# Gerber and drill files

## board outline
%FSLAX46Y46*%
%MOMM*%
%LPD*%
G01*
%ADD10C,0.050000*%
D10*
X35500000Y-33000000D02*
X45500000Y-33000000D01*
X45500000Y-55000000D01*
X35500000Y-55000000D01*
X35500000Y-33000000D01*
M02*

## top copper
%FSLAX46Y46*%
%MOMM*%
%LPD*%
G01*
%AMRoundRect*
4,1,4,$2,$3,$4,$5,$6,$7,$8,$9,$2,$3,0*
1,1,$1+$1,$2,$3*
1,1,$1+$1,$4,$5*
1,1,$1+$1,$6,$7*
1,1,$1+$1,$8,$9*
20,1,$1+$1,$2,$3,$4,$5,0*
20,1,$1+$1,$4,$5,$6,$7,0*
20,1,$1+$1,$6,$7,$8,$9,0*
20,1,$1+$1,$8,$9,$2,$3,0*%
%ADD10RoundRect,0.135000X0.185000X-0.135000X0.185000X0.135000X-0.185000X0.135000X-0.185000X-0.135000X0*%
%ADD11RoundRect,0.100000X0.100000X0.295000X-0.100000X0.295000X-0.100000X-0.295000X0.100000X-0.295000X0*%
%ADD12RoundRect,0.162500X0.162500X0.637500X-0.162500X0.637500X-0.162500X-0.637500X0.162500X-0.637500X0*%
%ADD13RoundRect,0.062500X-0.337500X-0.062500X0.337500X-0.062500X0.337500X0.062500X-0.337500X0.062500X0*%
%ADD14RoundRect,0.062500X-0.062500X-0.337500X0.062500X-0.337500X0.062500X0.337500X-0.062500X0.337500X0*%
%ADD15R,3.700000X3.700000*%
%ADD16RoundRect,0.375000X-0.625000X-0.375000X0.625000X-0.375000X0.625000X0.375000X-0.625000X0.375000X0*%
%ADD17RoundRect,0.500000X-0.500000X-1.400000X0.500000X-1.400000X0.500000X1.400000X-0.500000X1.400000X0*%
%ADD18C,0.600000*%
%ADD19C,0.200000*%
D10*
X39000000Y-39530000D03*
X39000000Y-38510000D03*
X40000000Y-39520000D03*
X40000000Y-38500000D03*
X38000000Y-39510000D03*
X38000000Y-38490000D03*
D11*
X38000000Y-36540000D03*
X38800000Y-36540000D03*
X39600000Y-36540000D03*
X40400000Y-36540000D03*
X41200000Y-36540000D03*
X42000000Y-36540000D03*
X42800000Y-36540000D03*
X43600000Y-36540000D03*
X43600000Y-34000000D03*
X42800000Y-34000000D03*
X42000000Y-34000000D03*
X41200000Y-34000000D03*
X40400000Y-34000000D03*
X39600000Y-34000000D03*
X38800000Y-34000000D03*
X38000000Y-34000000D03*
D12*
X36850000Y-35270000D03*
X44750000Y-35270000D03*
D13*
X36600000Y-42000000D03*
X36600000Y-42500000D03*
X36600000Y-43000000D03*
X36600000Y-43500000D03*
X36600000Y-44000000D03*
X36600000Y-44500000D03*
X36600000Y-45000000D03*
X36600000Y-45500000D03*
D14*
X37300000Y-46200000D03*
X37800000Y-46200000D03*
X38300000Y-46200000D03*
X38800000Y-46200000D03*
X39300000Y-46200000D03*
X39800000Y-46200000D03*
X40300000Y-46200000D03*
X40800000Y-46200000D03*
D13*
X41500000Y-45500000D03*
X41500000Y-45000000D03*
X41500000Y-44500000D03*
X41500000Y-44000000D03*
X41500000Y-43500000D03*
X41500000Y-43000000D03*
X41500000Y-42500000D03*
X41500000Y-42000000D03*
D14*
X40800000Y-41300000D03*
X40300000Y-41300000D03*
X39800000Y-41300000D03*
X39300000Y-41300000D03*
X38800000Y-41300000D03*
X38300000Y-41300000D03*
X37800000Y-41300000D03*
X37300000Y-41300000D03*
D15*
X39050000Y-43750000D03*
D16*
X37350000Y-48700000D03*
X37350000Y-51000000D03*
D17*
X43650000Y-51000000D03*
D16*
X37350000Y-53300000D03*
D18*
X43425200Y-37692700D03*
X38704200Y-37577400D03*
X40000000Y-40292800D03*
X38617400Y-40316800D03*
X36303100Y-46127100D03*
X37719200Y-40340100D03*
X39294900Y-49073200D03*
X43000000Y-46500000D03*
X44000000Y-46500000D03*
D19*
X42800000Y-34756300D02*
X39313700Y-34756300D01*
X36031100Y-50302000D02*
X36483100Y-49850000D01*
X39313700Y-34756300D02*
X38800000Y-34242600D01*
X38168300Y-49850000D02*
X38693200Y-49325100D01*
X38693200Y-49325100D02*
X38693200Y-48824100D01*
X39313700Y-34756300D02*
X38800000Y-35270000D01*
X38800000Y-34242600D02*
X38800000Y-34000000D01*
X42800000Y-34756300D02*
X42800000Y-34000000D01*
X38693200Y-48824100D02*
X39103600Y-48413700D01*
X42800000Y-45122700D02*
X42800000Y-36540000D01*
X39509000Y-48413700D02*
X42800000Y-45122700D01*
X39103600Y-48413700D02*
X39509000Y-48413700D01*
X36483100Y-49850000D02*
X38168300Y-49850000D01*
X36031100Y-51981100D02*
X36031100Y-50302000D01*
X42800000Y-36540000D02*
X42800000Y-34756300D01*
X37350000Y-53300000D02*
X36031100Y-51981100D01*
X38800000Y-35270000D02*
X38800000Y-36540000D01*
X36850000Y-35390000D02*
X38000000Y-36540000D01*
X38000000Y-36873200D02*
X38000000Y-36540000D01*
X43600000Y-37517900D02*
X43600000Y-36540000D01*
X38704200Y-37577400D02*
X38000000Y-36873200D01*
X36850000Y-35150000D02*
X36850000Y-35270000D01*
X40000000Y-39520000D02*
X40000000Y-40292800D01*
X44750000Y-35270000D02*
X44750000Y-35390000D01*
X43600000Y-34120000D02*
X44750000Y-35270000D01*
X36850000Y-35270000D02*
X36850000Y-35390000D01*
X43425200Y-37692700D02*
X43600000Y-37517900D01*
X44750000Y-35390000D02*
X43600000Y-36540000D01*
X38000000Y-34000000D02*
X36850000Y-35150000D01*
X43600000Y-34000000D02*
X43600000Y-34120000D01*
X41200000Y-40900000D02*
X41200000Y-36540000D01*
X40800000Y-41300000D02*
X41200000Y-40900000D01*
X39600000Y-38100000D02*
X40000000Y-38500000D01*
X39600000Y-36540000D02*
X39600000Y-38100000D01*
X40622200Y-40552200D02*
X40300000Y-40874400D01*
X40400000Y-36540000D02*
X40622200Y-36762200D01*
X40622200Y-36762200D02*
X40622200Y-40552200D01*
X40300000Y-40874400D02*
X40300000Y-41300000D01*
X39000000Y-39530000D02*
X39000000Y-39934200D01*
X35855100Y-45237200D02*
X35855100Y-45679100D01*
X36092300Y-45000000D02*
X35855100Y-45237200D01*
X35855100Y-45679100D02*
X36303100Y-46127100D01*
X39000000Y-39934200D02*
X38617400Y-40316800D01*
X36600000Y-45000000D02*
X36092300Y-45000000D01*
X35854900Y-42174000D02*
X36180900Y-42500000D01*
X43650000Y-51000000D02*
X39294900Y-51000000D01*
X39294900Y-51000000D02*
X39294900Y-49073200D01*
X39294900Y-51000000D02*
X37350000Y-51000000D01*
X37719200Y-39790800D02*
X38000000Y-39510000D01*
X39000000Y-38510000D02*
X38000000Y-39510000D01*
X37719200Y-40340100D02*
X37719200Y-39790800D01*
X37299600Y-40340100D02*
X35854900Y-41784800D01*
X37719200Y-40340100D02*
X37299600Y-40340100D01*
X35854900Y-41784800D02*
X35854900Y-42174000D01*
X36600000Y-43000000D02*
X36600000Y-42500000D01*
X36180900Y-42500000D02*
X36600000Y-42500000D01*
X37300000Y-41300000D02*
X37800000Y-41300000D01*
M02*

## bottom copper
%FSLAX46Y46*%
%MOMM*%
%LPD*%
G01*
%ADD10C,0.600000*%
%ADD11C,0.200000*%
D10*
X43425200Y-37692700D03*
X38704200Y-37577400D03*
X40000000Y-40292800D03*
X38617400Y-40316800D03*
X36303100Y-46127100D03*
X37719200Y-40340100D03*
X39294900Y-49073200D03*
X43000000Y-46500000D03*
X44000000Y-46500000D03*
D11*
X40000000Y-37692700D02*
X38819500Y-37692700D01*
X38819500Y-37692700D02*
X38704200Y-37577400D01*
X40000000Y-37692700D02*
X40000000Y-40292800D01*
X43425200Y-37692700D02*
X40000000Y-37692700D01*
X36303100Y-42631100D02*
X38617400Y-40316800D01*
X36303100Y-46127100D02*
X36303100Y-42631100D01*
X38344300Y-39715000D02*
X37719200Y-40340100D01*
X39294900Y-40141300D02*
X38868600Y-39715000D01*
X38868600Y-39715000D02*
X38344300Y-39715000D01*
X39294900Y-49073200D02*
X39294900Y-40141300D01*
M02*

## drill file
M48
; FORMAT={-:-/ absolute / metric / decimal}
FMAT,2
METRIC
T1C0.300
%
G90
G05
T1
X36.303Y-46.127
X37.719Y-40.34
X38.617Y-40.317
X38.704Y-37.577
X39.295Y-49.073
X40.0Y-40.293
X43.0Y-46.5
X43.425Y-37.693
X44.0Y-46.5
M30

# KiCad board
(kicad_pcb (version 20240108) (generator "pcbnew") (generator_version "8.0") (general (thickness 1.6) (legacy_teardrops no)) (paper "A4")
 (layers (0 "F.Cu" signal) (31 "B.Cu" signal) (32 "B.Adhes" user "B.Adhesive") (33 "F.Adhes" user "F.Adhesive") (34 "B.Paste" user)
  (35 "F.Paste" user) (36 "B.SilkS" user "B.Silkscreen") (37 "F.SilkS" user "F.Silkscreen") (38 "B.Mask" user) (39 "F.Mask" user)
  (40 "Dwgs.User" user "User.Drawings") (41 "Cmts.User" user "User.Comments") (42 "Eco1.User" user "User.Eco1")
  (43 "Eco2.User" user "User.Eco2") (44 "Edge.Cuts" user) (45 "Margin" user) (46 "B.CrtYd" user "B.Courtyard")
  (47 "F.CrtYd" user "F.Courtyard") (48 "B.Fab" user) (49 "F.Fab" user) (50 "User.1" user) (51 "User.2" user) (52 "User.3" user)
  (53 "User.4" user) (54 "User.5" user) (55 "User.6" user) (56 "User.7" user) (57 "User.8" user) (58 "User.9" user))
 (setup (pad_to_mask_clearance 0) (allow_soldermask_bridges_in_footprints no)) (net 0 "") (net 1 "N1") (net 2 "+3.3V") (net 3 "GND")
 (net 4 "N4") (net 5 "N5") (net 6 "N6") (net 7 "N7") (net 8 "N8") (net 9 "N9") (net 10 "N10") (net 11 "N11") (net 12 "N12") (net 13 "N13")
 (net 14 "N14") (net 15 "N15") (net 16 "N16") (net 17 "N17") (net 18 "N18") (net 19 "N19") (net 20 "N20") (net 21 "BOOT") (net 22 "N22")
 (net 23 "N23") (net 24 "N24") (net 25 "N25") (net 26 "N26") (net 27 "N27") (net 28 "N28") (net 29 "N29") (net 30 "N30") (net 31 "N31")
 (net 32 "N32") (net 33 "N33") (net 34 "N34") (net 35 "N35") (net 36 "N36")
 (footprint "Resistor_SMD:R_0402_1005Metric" (layer "F.Cu") (at 39 39.02 90)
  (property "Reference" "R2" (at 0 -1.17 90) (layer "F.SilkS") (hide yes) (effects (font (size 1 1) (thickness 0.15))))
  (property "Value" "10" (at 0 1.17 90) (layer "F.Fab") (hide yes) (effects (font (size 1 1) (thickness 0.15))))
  (pad "1" smd roundrect (at -0.51 0 90) (size 0.54 0.64) (layers "F.Cu" "F.Paste" "F.Mask") (roundrect_rratio 0.25) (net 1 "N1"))
  (pad "2" smd roundrect (at 0.51 0 90) (size 0.54 0.64) (layers "F.Cu" "F.Paste" "F.Mask") (roundrect_rratio 0.25) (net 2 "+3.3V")))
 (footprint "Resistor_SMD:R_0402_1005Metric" (layer "F.Cu") (at 40 39.01 90)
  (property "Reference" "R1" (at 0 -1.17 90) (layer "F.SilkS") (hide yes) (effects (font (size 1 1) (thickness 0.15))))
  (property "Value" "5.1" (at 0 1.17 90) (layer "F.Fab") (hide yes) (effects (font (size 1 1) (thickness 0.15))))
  (pad "1" smd roundrect (at -0.51 0 90) (size 0.54 0.64) (layers "F.Cu" "F.Paste" "F.Mask") (roundrect_rratio 0.25) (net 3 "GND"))
  (pad "2" smd roundrect (at 0.51 0 90) (size 0.54 0.64) (layers "F.Cu" "F.Paste" "F.Mask") (roundrect_rratio 0.25) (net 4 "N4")))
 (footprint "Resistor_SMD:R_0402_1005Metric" (layer "F.Cu") (at 38 39 90)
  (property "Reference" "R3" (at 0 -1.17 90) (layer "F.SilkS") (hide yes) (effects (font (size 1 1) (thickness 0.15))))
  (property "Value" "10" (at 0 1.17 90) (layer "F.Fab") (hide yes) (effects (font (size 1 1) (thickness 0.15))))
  (pad "1" smd roundrect (at -0.51 0 90) (size 0.54 0.64) (layers "F.Cu" "F.Paste" "F.Mask") (roundrect_rratio 0.25) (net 2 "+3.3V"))
  (pad "2" smd roundrect (at 0.51 0 90) (size 0.54 0.64) (layers "F.Cu" "F.Paste" "F.Mask") (roundrect_rratio 0.25) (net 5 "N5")))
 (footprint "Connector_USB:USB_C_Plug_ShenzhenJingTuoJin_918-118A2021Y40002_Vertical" (layer "F.Cu") (at 40.8 35.27 90)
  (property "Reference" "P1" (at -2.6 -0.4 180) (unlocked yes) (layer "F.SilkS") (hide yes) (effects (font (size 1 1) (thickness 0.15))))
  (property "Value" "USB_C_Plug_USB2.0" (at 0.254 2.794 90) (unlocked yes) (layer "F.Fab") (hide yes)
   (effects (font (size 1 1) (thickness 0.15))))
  (pad "A1" smd roundrect (at -1.27 -2.8 180) (size 0.4 0.79) (layers "F.Cu" "F.Paste" "F.Mask") (roundrect_rratio 0.25) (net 3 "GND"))
  (pad "A4" smd roundrect (at -1.27 -2 180) (size 0.4 0.79) (layers "F.Cu" "F.Paste" "F.Mask") (roundrect_rratio 0.25) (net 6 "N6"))
  (pad "A5" smd roundrect (at -1.27 -1.2 180) (size 0.4 0.79) (layers "F.Cu" "F.Paste" "F.Mask") (roundrect_rratio 0.25) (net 4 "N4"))
  (pad "A6" smd roundrect (at -1.27 -0.4 180) (size 0.4 0.79) (layers "F.Cu" "F.Paste" "F.Mask") (roundrect_rratio 0.25) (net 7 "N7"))
  (pad "A7" smd roundrect (at -1.27 0.4 180) (size 0.4 0.79) (layers "F.Cu" "F.Paste" "F.Mask") (roundrect_rratio 0.25) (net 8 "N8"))
  (pad "A8" smd roundrect (at -1.27 1.2 180) (size 0.4 0.79) (layers "F.Cu" "F.Paste" "F.Mask") (roundrect_rratio 0.25))
  (pad "A9" smd roundrect (at -1.27 2 180) (size 0.4 0.79) (layers "F.Cu" "F.Paste" "F.Mask") (roundrect_rratio 0.25) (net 6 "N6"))
  (pad "A12" smd roundrect (at -1.27 2.8 180) (size 0.4 0.79) (layers "F.Cu" "F.Paste" "F.Mask") (roundrect_rratio 0.25) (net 3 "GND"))
  (pad "B1" smd roundrect (at 1.27 2.8 180) (size 0.4 0.79) (layers "F.Cu" "F.Paste" "F.Mask") (roundrect_rratio 0.25) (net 3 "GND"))
  (pad "B4" smd roundrect (at 1.27 2 180) (size 0.4 0.79) (layers "F.Cu" "F.Paste" "F.Mask") (roundrect_rratio 0.25) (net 6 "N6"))
  (pad "B5" smd roundrect (at 1.27 1.2 180) (size 0.4 0.79) (layers "F.Cu" "F.Paste" "F.Mask") (roundrect_rratio 0.25) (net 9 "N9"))
  (pad "B6" smd roundrect (at 1.27 0.4 180) (size 0.4 0.79) (layers "F.Cu" "F.Paste" "F.Mask") (roundrect_rratio 0.25))
  (pad "B7" smd roundrect (at 1.27 -0.4 180) (size 0.4 0.79) (layers "F.Cu" "F.Paste" "F.Mask") (roundrect_rratio 0.25))
  (pad "B8" smd roundrect (at 1.27 -1.2 180) (size 0.4 0.79) (layers "F.Cu" "F.Paste" "F.Mask") (roundrect_rratio 0.25))
  (pad "B9" smd roundrect (at 1.27 -2 180) (size 0.4 0.79) (layers "F.Cu" "F.Paste" "F.Mask") (roundrect_rratio 0.25) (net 6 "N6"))
  (pad "B12" smd roundrect (at 1.27 -2.8 180) (size 0.4 0.79) (layers "F.Cu" "F.Paste" "F.Mask") (roundrect_rratio 0.25) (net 3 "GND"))
  (pad "S1" smd roundrect (at 0 -3.95 180) (size 0.65 1.6) (layers "F.Cu" "F.Paste" "F.Mask") (roundrect_rratio 0.25) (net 3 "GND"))
  (pad "S1" smd roundrect (at 0 3.95 180) (size 0.65 1.6) (layers "F.Cu" "F.Paste" "F.Mask") (roundrect_rratio 0.25) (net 3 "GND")))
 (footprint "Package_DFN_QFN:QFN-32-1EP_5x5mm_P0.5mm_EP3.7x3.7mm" (layer "F.Cu") (at 39.05 43.75)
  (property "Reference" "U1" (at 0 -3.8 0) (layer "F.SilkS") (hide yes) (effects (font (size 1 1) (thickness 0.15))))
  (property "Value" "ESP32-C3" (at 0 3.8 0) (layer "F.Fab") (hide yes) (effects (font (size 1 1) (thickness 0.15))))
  (pad "" smd roundrect (at -0.925 -0.925) (size 1.49 1.49) (layers "F.Paste") (roundrect_rratio 0.167785))
  (pad "" smd roundrect (at -0.925 0.925) (size 1.49 1.49) (layers "F.Paste") (roundrect_rratio 0.167785))
  (pad "" smd roundrect (at 0.925 -0.925) (size 1.49 1.49) (layers "F.Paste") (roundrect_rratio 0.167785))
  (pad "" smd roundrect (at 0.925 0.925) (size 1.49 1.49) (layers "F.Paste") (roundrect_rratio 0.167785))
  (pad "1" smd roundrect (at -2.45 -1.75) (size 0.8 0.25) (layers "F.Cu" "F.Paste" "F.Mask") (roundrect_rratio 0.25) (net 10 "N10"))
  (pad "2" smd roundrect (at -2.45 -1.25) (size 0.8 0.25) (layers "F.Cu" "F.Paste" "F.Mask") (roundrect_rratio 0.25) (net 2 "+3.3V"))
  (pad "3" smd roundrect (at -2.45 -0.75) (size 0.8 0.25) (layers "F.Cu" "F.Paste" "F.Mask") (roundrect_rratio 0.25) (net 2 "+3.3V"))
  (pad "4" smd roundrect (at -2.45 -0.25) (size 0.8 0.25) (layers "F.Cu" "F.Paste" "F.Mask") (roundrect_rratio 0.25) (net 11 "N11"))
  (pad "5" smd roundrect (at -2.45 0.25) (size 0.8 0.25) (layers "F.Cu" "F.Paste" "F.Mask") (roundrect_rratio 0.25) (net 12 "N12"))
  (pad "6" smd roundrect (at -2.45 0.75) (size 0.8 0.25) (layers "F.Cu" "F.Paste" "F.Mask") (roundrect_rratio 0.25) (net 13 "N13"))
  (pad "7" smd roundrect (at -2.45 1.25) (size 0.8 0.25) (layers "F.Cu" "F.Paste" "F.Mask") (roundrect_rratio 0.25) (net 1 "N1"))
  (pad "8" smd roundrect (at -2.45 1.75) (size 0.8 0.25) (layers "F.Cu" "F.Paste" "F.Mask") (roundrect_rratio 0.25) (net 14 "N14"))
  (pad "9" smd roundrect (at -1.75 2.45) (size 0.25 0.8) (layers "F.Cu" "F.Paste" "F.Mask") (roundrect_rratio 0.25) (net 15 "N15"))
  (pad "10" smd roundrect (at -1.25 2.45) (size 0.25 0.8) (layers "F.Cu" "F.Paste" "F.Mask") (roundrect_rratio 0.25) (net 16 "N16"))
  (pad "11" smd roundrect (at -0.75 2.45) (size 0.25 0.8) (layers "F.Cu" "F.Paste" "F.Mask") (roundrect_rratio 0.25) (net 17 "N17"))
  (pad "12" smd roundrect (at -0.25 2.45) (size 0.25 0.8) (layers "F.Cu" "F.Paste" "F.Mask") (roundrect_rratio 0.25) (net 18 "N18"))
  (pad "13" smd roundrect (at 0.25 2.45) (size 0.25 0.8) (layers "F.Cu" "F.Paste" "F.Mask") (roundrect_rratio 0.25) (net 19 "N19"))
  (pad "14" smd roundrect (at 0.75 2.45) (size 0.25 0.8) (layers "F.Cu" "F.Paste" "F.Mask") (roundrect_rratio 0.25) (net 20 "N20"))
  (pad "15" smd roundrect (at 1.25 2.45) (size 0.25 0.8) (layers "F.Cu" "F.Paste" "F.Mask") (roundrect_rratio 0.25) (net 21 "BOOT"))
  (pad "16" smd roundrect (at 1.75 2.45) (size 0.25 0.8) (layers "F.Cu" "F.Paste" "F.Mask") (roundrect_rratio 0.25) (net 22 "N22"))
  (pad "17" smd roundrect (at 2.45 1.75) (size 0.8 0.25) (layers "F.Cu" "F.Paste" "F.Mask") (roundrect_rratio 0.25) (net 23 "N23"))
  (pad "18" smd roundrect (at 2.45 1.25) (size 0.8 0.25) (layers "F.Cu" "F.Paste" "F.Mask") (roundrect_rratio 0.25) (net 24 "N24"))
  (pad "19" smd roundrect (at 2.45 0.75) (size 0.8 0.25) (layers "F.Cu" "F.Paste" "F.Mask") (roundrect_rratio 0.25) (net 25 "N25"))
  (pad "20" smd roundrect (at 2.45 0.25) (size 0.8 0.25) (layers "F.Cu" "F.Paste" "F.Mask") (roundrect_rratio 0.25) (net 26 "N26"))
  (pad "21" smd roundrect (at 2.45 -0.25) (size 0.8 0.25) (layers "F.Cu" "F.Paste" "F.Mask") (roundrect_rratio 0.25) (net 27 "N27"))
  (pad "22" smd roundrect (at 2.45 -0.75) (size 0.8 0.25) (layers "F.Cu" "F.Paste" "F.Mask") (roundrect_rratio 0.25) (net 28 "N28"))
  (pad "23" smd roundrect (at 2.45 -1.25) (size 0.8 0.25) (layers "F.Cu" "F.Paste" "F.Mask") (roundrect_rratio 0.25) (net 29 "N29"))
  (pad "24" smd roundrect (at 2.45 -1.75) (size 0.8 0.25) (layers "F.Cu" "F.Paste" "F.Mask") (roundrect_rratio 0.25) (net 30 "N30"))
  (pad "25" smd roundrect (at 1.75 -2.45) (size 0.25 0.8) (layers "F.Cu" "F.Paste" "F.Mask") (roundrect_rratio 0.25) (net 8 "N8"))
  (pad "26" smd roundrect (at 1.25 -2.45) (size 0.25 0.8) (layers "F.Cu" "F.Paste" "F.Mask") (roundrect_rratio 0.25) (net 7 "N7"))
  (pad "27" smd roundrect (at 0.75 -2.45) (size 0.25 0.8) (layers "F.Cu" "F.Paste" "F.Mask") (roundrect_rratio 0.25) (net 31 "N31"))
  (pad "28" smd roundrect (at 0.25 -2.45) (size 0.25 0.8) (layers "F.Cu" "F.Paste" "F.Mask") (roundrect_rratio 0.25) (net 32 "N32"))
  (pad "29" smd roundrect (at -0.25 -2.45) (size 0.25 0.8) (layers "F.Cu" "F.Paste" "F.Mask") (roundrect_rratio 0.25) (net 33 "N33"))
  (pad "30" smd roundrect (at -0.75 -2.45) (size 0.25 0.8) (layers "F.Cu" "F.Paste" "F.Mask") (roundrect_rratio 0.25) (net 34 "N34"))
  (pad "31" smd roundrect (at -1.25 -2.45) (size 0.25 0.8) (layers "F.Cu" "F.Paste" "F.Mask") (roundrect_rratio 0.25) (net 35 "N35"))
  (pad "32" smd roundrect (at -1.75 -2.45) (size 0.25 0.8) (layers "F.Cu" "F.Paste" "F.Mask") (roundrect_rratio 0.25) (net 35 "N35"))
  (pad "33" smd rect (at 0 0) (size 3.7 3.7) (layers "F.Cu" "F.Mask") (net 3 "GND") (zone_connect 2)))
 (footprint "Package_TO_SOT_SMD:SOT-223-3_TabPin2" (layer "F.Cu") (at 40.5 51)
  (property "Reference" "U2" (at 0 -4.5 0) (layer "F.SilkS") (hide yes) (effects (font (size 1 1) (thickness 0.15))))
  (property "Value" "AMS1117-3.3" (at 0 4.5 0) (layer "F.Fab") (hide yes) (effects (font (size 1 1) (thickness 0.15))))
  (pad "1" smd roundrect (at -3.15 -2.3) (size 2 1.5) (layers "F.Cu" "F.Paste" "F.Mask") (roundrect_rratio 0.25) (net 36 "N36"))
  (pad "2" smd roundrect (at -3.15 0) (size 2 1.5) (layers "F.Cu" "F.Paste" "F.Mask") (roundrect_rratio 0.25) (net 2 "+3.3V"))
  (pad "2" smd roundrect (at 3.15 0) (size 2 3.8) (layers "F.Cu" "F.Paste" "F.Mask") (roundrect_rratio 0.25) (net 2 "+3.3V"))
  (pad "3" smd roundrect (at -3.15 2.3) (size 2 1.5) (layers "F.Cu" "F.Paste" "F.Mask") (roundrect_rratio 0.25) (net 6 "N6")))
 (gr_rect (start 35.5 33) (end 45.5 55) (stroke (width 0.05) (type default)) (fill none) (layer "Edge.Cuts"))
 (segment (start 42.8 34.7563) (end 39.3137 34.7563) (width 0.2) (layer "F.Cu") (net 6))
 (segment (start 36.0311 50.302) (end 36.4831 49.85) (width 0.2) (layer "F.Cu") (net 6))
 (segment (start 39.3137 34.7563) (end 38.8 34.2426) (width 0.2) (layer "F.Cu") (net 6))
 (segment (start 38.1683 49.85) (end 38.6932 49.3251) (width 0.2) (layer "F.Cu") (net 6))
 (segment (start 38.6932 49.3251) (end 38.6932 48.8241) (width 0.2) (layer "F.Cu") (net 6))
 (segment (start 39.3137 34.7563) (end 38.8 35.27) (width 0.2) (layer "F.Cu") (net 6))
 (segment (start 38.8 34.2426) (end 38.8 34) (width 0.2) (layer "F.Cu") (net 6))
 (segment (start 42.8 34.7563) (end 42.8 34) (width 0.2) (layer "F.Cu") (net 6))
 (segment (start 38.6932 48.8241) (end 39.1036 48.4137) (width 0.2) (layer "F.Cu") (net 6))
 (segment (start 42.8 45.1227) (end 42.8 36.54) (width 0.2) (layer "F.Cu") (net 6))
 (segment (start 39.509 48.4137) (end 42.8 45.1227) (width 0.2) (layer "F.Cu") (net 6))
 (segment (start 39.1036 48.4137) (end 39.509 48.4137) (width 0.2) (layer "F.Cu") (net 6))
 (segment (start 36.4831 49.85) (end 38.1683 49.85) (width 0.2) (layer "F.Cu") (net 6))
 (segment (start 36.0311 51.9811) (end 36.0311 50.302) (width 0.2) (layer "F.Cu") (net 6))
 (segment (start 42.8 36.54) (end 42.8 34.7563) (width 0.2) (layer "F.Cu") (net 6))
 (segment (start 37.35 53.3) (end 36.0311 51.9811) (width 0.2) (layer "F.Cu") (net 6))
 (segment (start 38.8 35.27) (end 38.8 36.54) (width 0.2) (layer "F.Cu") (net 6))
 (segment (start 36.85 35.39) (end 38 36.54) (width 0.2) (layer "F.Cu") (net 3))
 (segment (start 38 36.8732) (end 38 36.54) (width 0.2) (layer "F.Cu") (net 3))
 (segment (start 43.6 37.5179) (end 43.6 36.54) (width 0.2) (layer "F.Cu") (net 3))
 (segment (start 38.7042 37.5774) (end 38 36.8732) (width 0.2) (layer "F.Cu") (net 3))
 (segment (start 36.85 35.15) (end 36.85 35.27) (width 0.2) (layer "F.Cu") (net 3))
 (segment (start 40 39.52) (end 40 40.2928) (width 0.2) (layer "F.Cu") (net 3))
 (segment (start 44.75 35.27) (end 44.75 35.39) (width 0.2) (layer "F.Cu") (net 3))
 (segment (start 43.6 34.12) (end 44.75 35.27) (width 0.2) (layer "F.Cu") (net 3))
 (segment (start 36.85 35.27) (end 36.85 35.39) (width 0.2) (layer "F.Cu") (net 3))
 (segment (start 43.4252 37.6927) (end 43.6 37.5179) (width 0.2) (layer "F.Cu") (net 3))
 (segment (start 44.75 35.39) (end 43.6 36.54) (width 0.2) (layer "F.Cu") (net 3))
 (segment (start 38 34) (end 36.85 35.15) (width 0.2) (layer "F.Cu") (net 3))
 (segment (start 43.6 34) (end 43.6 34.12) (width 0.2) (layer "F.Cu") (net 3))
 (via (at 43.4252 37.6927) (size 0.6) (drill 0.3) (layers "F.Cu" "B.Cu") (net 3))
 (via (at 38.7042 37.5774) (size 0.6) (drill 0.3) (layers "F.Cu" "B.Cu") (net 3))
 (via (at 40 40.2928) (size 0.6) (drill 0.3) (layers "F.Cu" "B.Cu") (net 3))
 (segment (start 40 37.6927) (end 38.8195 37.6927) (width 0.2) (layer "B.Cu") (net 3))
 (segment (start 38.8195 37.6927) (end 38.7042 37.5774) (width 0.2) (layer "B.Cu") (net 3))
 (segment (start 40 37.6927) (end 40 40.2928) (width 0.2) (layer "B.Cu") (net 3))
 (segment (start 43.4252 37.6927) (end 40 37.6927) (width 0.2) (layer "B.Cu") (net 3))
 (segment (start 41.2 40.9) (end 41.2 36.54) (width 0.2) (layer "F.Cu") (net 8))
 (segment (start 40.8 41.3) (end 41.2 40.9) (width 0.2) (layer "F.Cu") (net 8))
 (segment (start 39.6 38.1) (end 40 38.5) (width 0.2) (layer "F.Cu") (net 4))
 (segment (start 39.6 36.54) (end 39.6 38.1) (width 0.2) (layer "F.Cu") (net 4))
 (segment (start 40.6222 40.5522) (end 40.3 40.8744) (width 0.2) (layer "F.Cu") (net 7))
 (segment (start 40.4 36.54) (end 40.6222 36.7622) (width 0.2) (layer "F.Cu") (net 7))
 (segment (start 40.6222 36.7622) (end 40.6222 40.5522) (width 0.2) (layer "F.Cu") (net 7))
 (segment (start 40.3 40.8744) (end 40.3 41.3) (width 0.2) (layer "F.Cu") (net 7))
 (segment (start 39 39.53) (end 39 39.9342) (width 0.2) (layer "F.Cu") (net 1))
 (segment (start 35.8551 45.2372) (end 35.8551 45.6791) (width 0.2) (layer "F.Cu") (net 1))
 (segment (start 36.0923 45) (end 35.8551 45.2372) (width 0.2) (layer "F.Cu") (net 1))
 (segment (start 35.8551 45.6791) (end 36.3031 46.1271) (width 0.2) (layer "F.Cu") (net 1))
 (segment (start 39 39.9342) (end 38.6174 40.3168) (width 0.2) (layer "F.Cu") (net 1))
 (segment (start 36.6 45) (end 36.0923 45) (width 0.2) (layer "F.Cu") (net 1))
 (via (at 38.6174 40.3168) (size 0.6) (drill 0.3) (layers "F.Cu" "B.Cu") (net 1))
 (via (at 36.3031 46.1271) (size 0.6) (drill 0.3) (layers "F.Cu" "B.Cu") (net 1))
 (segment (start 36.3031 42.6311) (end 38.6174 40.3168) (width 0.2) (layer "B.Cu") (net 1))
 (segment (start 36.3031 46.1271) (end 36.3031 42.6311) (width 0.2) (layer "B.Cu") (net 1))
 (segment (start 35.8549 42.174) (end 36.1809 42.5) (width 0.2) (layer "F.Cu") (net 2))
 (segment (start 43.65 51) (end 39.2949 51) (width 0.2) (layer "F.Cu") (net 2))
 (segment (start 39.2949 51) (end 39.2949 49.0732) (width 0.2) (layer "F.Cu") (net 2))
 (segment (start 39.2949 51) (end 37.35 51) (width 0.2) (layer "F.Cu") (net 2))
 (segment (start 37.7192 39.7908) (end 38 39.51) (width 0.2) (layer "F.Cu") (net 2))
 (segment (start 39 38.51) (end 38 39.51) (width 0.2) (layer "F.Cu") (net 2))
 (segment (start 37.7192 40.3401) (end 37.7192 39.7908) (width 0.2) (layer "F.Cu") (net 2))
 (segment (start 37.2996 40.3401) (end 35.8549 41.7848) (width 0.2) (layer "F.Cu") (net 2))
 (segment (start 37.7192 40.3401) (end 37.2996 40.3401) (width 0.2) (layer "F.Cu") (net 2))
 (segment (start 35.8549 41.7848) (end 35.8549 42.174) (width 0.2) (layer "F.Cu") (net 2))
 (segment (start 36.6 43) (end 36.6 42.5) (width 0.2) (layer "F.Cu") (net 2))
 (segment (start 36.1809 42.5) (end 36.6 42.5) (width 0.2) (layer "F.Cu") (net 2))
 (via (at 37.7192 40.3401) (size 0.6) (drill 0.3) (layers "F.Cu" "B.Cu") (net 2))
 (via (at 39.2949 49.0732) (size 0.6) (drill 0.3) (layers "F.Cu" "B.Cu") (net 2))
 (segment (start 38.3443 39.715) (end 37.7192 40.3401) (width 0.2) (layer "B.Cu") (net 2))
 (segment (start 39.2949 40.1413) (end 38.8686 39.715) (width 0.2) (layer "B.Cu") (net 2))
 (segment (start 38.8686 39.715) (end 38.3443 39.715) (width 0.2) (layer "B.Cu") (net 2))
 (segment (start 39.2949 49.0732) (end 39.2949 40.1413) (width 0.2) (layer "B.Cu") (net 2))
 (via (at 43 46.5) (size 0.6) (drill 0.3) (layers "F.Cu" "B.Cu") (free yes) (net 21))
 (segment (start 37.3 41.3) (end 37.8 41.3) (width 0.2) (layer "F.Cu") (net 35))
 (via (at 44 46.5) (size 0.6) (drill 0.3) (layers "F.Cu" "B.Cu") (free yes) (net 5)))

